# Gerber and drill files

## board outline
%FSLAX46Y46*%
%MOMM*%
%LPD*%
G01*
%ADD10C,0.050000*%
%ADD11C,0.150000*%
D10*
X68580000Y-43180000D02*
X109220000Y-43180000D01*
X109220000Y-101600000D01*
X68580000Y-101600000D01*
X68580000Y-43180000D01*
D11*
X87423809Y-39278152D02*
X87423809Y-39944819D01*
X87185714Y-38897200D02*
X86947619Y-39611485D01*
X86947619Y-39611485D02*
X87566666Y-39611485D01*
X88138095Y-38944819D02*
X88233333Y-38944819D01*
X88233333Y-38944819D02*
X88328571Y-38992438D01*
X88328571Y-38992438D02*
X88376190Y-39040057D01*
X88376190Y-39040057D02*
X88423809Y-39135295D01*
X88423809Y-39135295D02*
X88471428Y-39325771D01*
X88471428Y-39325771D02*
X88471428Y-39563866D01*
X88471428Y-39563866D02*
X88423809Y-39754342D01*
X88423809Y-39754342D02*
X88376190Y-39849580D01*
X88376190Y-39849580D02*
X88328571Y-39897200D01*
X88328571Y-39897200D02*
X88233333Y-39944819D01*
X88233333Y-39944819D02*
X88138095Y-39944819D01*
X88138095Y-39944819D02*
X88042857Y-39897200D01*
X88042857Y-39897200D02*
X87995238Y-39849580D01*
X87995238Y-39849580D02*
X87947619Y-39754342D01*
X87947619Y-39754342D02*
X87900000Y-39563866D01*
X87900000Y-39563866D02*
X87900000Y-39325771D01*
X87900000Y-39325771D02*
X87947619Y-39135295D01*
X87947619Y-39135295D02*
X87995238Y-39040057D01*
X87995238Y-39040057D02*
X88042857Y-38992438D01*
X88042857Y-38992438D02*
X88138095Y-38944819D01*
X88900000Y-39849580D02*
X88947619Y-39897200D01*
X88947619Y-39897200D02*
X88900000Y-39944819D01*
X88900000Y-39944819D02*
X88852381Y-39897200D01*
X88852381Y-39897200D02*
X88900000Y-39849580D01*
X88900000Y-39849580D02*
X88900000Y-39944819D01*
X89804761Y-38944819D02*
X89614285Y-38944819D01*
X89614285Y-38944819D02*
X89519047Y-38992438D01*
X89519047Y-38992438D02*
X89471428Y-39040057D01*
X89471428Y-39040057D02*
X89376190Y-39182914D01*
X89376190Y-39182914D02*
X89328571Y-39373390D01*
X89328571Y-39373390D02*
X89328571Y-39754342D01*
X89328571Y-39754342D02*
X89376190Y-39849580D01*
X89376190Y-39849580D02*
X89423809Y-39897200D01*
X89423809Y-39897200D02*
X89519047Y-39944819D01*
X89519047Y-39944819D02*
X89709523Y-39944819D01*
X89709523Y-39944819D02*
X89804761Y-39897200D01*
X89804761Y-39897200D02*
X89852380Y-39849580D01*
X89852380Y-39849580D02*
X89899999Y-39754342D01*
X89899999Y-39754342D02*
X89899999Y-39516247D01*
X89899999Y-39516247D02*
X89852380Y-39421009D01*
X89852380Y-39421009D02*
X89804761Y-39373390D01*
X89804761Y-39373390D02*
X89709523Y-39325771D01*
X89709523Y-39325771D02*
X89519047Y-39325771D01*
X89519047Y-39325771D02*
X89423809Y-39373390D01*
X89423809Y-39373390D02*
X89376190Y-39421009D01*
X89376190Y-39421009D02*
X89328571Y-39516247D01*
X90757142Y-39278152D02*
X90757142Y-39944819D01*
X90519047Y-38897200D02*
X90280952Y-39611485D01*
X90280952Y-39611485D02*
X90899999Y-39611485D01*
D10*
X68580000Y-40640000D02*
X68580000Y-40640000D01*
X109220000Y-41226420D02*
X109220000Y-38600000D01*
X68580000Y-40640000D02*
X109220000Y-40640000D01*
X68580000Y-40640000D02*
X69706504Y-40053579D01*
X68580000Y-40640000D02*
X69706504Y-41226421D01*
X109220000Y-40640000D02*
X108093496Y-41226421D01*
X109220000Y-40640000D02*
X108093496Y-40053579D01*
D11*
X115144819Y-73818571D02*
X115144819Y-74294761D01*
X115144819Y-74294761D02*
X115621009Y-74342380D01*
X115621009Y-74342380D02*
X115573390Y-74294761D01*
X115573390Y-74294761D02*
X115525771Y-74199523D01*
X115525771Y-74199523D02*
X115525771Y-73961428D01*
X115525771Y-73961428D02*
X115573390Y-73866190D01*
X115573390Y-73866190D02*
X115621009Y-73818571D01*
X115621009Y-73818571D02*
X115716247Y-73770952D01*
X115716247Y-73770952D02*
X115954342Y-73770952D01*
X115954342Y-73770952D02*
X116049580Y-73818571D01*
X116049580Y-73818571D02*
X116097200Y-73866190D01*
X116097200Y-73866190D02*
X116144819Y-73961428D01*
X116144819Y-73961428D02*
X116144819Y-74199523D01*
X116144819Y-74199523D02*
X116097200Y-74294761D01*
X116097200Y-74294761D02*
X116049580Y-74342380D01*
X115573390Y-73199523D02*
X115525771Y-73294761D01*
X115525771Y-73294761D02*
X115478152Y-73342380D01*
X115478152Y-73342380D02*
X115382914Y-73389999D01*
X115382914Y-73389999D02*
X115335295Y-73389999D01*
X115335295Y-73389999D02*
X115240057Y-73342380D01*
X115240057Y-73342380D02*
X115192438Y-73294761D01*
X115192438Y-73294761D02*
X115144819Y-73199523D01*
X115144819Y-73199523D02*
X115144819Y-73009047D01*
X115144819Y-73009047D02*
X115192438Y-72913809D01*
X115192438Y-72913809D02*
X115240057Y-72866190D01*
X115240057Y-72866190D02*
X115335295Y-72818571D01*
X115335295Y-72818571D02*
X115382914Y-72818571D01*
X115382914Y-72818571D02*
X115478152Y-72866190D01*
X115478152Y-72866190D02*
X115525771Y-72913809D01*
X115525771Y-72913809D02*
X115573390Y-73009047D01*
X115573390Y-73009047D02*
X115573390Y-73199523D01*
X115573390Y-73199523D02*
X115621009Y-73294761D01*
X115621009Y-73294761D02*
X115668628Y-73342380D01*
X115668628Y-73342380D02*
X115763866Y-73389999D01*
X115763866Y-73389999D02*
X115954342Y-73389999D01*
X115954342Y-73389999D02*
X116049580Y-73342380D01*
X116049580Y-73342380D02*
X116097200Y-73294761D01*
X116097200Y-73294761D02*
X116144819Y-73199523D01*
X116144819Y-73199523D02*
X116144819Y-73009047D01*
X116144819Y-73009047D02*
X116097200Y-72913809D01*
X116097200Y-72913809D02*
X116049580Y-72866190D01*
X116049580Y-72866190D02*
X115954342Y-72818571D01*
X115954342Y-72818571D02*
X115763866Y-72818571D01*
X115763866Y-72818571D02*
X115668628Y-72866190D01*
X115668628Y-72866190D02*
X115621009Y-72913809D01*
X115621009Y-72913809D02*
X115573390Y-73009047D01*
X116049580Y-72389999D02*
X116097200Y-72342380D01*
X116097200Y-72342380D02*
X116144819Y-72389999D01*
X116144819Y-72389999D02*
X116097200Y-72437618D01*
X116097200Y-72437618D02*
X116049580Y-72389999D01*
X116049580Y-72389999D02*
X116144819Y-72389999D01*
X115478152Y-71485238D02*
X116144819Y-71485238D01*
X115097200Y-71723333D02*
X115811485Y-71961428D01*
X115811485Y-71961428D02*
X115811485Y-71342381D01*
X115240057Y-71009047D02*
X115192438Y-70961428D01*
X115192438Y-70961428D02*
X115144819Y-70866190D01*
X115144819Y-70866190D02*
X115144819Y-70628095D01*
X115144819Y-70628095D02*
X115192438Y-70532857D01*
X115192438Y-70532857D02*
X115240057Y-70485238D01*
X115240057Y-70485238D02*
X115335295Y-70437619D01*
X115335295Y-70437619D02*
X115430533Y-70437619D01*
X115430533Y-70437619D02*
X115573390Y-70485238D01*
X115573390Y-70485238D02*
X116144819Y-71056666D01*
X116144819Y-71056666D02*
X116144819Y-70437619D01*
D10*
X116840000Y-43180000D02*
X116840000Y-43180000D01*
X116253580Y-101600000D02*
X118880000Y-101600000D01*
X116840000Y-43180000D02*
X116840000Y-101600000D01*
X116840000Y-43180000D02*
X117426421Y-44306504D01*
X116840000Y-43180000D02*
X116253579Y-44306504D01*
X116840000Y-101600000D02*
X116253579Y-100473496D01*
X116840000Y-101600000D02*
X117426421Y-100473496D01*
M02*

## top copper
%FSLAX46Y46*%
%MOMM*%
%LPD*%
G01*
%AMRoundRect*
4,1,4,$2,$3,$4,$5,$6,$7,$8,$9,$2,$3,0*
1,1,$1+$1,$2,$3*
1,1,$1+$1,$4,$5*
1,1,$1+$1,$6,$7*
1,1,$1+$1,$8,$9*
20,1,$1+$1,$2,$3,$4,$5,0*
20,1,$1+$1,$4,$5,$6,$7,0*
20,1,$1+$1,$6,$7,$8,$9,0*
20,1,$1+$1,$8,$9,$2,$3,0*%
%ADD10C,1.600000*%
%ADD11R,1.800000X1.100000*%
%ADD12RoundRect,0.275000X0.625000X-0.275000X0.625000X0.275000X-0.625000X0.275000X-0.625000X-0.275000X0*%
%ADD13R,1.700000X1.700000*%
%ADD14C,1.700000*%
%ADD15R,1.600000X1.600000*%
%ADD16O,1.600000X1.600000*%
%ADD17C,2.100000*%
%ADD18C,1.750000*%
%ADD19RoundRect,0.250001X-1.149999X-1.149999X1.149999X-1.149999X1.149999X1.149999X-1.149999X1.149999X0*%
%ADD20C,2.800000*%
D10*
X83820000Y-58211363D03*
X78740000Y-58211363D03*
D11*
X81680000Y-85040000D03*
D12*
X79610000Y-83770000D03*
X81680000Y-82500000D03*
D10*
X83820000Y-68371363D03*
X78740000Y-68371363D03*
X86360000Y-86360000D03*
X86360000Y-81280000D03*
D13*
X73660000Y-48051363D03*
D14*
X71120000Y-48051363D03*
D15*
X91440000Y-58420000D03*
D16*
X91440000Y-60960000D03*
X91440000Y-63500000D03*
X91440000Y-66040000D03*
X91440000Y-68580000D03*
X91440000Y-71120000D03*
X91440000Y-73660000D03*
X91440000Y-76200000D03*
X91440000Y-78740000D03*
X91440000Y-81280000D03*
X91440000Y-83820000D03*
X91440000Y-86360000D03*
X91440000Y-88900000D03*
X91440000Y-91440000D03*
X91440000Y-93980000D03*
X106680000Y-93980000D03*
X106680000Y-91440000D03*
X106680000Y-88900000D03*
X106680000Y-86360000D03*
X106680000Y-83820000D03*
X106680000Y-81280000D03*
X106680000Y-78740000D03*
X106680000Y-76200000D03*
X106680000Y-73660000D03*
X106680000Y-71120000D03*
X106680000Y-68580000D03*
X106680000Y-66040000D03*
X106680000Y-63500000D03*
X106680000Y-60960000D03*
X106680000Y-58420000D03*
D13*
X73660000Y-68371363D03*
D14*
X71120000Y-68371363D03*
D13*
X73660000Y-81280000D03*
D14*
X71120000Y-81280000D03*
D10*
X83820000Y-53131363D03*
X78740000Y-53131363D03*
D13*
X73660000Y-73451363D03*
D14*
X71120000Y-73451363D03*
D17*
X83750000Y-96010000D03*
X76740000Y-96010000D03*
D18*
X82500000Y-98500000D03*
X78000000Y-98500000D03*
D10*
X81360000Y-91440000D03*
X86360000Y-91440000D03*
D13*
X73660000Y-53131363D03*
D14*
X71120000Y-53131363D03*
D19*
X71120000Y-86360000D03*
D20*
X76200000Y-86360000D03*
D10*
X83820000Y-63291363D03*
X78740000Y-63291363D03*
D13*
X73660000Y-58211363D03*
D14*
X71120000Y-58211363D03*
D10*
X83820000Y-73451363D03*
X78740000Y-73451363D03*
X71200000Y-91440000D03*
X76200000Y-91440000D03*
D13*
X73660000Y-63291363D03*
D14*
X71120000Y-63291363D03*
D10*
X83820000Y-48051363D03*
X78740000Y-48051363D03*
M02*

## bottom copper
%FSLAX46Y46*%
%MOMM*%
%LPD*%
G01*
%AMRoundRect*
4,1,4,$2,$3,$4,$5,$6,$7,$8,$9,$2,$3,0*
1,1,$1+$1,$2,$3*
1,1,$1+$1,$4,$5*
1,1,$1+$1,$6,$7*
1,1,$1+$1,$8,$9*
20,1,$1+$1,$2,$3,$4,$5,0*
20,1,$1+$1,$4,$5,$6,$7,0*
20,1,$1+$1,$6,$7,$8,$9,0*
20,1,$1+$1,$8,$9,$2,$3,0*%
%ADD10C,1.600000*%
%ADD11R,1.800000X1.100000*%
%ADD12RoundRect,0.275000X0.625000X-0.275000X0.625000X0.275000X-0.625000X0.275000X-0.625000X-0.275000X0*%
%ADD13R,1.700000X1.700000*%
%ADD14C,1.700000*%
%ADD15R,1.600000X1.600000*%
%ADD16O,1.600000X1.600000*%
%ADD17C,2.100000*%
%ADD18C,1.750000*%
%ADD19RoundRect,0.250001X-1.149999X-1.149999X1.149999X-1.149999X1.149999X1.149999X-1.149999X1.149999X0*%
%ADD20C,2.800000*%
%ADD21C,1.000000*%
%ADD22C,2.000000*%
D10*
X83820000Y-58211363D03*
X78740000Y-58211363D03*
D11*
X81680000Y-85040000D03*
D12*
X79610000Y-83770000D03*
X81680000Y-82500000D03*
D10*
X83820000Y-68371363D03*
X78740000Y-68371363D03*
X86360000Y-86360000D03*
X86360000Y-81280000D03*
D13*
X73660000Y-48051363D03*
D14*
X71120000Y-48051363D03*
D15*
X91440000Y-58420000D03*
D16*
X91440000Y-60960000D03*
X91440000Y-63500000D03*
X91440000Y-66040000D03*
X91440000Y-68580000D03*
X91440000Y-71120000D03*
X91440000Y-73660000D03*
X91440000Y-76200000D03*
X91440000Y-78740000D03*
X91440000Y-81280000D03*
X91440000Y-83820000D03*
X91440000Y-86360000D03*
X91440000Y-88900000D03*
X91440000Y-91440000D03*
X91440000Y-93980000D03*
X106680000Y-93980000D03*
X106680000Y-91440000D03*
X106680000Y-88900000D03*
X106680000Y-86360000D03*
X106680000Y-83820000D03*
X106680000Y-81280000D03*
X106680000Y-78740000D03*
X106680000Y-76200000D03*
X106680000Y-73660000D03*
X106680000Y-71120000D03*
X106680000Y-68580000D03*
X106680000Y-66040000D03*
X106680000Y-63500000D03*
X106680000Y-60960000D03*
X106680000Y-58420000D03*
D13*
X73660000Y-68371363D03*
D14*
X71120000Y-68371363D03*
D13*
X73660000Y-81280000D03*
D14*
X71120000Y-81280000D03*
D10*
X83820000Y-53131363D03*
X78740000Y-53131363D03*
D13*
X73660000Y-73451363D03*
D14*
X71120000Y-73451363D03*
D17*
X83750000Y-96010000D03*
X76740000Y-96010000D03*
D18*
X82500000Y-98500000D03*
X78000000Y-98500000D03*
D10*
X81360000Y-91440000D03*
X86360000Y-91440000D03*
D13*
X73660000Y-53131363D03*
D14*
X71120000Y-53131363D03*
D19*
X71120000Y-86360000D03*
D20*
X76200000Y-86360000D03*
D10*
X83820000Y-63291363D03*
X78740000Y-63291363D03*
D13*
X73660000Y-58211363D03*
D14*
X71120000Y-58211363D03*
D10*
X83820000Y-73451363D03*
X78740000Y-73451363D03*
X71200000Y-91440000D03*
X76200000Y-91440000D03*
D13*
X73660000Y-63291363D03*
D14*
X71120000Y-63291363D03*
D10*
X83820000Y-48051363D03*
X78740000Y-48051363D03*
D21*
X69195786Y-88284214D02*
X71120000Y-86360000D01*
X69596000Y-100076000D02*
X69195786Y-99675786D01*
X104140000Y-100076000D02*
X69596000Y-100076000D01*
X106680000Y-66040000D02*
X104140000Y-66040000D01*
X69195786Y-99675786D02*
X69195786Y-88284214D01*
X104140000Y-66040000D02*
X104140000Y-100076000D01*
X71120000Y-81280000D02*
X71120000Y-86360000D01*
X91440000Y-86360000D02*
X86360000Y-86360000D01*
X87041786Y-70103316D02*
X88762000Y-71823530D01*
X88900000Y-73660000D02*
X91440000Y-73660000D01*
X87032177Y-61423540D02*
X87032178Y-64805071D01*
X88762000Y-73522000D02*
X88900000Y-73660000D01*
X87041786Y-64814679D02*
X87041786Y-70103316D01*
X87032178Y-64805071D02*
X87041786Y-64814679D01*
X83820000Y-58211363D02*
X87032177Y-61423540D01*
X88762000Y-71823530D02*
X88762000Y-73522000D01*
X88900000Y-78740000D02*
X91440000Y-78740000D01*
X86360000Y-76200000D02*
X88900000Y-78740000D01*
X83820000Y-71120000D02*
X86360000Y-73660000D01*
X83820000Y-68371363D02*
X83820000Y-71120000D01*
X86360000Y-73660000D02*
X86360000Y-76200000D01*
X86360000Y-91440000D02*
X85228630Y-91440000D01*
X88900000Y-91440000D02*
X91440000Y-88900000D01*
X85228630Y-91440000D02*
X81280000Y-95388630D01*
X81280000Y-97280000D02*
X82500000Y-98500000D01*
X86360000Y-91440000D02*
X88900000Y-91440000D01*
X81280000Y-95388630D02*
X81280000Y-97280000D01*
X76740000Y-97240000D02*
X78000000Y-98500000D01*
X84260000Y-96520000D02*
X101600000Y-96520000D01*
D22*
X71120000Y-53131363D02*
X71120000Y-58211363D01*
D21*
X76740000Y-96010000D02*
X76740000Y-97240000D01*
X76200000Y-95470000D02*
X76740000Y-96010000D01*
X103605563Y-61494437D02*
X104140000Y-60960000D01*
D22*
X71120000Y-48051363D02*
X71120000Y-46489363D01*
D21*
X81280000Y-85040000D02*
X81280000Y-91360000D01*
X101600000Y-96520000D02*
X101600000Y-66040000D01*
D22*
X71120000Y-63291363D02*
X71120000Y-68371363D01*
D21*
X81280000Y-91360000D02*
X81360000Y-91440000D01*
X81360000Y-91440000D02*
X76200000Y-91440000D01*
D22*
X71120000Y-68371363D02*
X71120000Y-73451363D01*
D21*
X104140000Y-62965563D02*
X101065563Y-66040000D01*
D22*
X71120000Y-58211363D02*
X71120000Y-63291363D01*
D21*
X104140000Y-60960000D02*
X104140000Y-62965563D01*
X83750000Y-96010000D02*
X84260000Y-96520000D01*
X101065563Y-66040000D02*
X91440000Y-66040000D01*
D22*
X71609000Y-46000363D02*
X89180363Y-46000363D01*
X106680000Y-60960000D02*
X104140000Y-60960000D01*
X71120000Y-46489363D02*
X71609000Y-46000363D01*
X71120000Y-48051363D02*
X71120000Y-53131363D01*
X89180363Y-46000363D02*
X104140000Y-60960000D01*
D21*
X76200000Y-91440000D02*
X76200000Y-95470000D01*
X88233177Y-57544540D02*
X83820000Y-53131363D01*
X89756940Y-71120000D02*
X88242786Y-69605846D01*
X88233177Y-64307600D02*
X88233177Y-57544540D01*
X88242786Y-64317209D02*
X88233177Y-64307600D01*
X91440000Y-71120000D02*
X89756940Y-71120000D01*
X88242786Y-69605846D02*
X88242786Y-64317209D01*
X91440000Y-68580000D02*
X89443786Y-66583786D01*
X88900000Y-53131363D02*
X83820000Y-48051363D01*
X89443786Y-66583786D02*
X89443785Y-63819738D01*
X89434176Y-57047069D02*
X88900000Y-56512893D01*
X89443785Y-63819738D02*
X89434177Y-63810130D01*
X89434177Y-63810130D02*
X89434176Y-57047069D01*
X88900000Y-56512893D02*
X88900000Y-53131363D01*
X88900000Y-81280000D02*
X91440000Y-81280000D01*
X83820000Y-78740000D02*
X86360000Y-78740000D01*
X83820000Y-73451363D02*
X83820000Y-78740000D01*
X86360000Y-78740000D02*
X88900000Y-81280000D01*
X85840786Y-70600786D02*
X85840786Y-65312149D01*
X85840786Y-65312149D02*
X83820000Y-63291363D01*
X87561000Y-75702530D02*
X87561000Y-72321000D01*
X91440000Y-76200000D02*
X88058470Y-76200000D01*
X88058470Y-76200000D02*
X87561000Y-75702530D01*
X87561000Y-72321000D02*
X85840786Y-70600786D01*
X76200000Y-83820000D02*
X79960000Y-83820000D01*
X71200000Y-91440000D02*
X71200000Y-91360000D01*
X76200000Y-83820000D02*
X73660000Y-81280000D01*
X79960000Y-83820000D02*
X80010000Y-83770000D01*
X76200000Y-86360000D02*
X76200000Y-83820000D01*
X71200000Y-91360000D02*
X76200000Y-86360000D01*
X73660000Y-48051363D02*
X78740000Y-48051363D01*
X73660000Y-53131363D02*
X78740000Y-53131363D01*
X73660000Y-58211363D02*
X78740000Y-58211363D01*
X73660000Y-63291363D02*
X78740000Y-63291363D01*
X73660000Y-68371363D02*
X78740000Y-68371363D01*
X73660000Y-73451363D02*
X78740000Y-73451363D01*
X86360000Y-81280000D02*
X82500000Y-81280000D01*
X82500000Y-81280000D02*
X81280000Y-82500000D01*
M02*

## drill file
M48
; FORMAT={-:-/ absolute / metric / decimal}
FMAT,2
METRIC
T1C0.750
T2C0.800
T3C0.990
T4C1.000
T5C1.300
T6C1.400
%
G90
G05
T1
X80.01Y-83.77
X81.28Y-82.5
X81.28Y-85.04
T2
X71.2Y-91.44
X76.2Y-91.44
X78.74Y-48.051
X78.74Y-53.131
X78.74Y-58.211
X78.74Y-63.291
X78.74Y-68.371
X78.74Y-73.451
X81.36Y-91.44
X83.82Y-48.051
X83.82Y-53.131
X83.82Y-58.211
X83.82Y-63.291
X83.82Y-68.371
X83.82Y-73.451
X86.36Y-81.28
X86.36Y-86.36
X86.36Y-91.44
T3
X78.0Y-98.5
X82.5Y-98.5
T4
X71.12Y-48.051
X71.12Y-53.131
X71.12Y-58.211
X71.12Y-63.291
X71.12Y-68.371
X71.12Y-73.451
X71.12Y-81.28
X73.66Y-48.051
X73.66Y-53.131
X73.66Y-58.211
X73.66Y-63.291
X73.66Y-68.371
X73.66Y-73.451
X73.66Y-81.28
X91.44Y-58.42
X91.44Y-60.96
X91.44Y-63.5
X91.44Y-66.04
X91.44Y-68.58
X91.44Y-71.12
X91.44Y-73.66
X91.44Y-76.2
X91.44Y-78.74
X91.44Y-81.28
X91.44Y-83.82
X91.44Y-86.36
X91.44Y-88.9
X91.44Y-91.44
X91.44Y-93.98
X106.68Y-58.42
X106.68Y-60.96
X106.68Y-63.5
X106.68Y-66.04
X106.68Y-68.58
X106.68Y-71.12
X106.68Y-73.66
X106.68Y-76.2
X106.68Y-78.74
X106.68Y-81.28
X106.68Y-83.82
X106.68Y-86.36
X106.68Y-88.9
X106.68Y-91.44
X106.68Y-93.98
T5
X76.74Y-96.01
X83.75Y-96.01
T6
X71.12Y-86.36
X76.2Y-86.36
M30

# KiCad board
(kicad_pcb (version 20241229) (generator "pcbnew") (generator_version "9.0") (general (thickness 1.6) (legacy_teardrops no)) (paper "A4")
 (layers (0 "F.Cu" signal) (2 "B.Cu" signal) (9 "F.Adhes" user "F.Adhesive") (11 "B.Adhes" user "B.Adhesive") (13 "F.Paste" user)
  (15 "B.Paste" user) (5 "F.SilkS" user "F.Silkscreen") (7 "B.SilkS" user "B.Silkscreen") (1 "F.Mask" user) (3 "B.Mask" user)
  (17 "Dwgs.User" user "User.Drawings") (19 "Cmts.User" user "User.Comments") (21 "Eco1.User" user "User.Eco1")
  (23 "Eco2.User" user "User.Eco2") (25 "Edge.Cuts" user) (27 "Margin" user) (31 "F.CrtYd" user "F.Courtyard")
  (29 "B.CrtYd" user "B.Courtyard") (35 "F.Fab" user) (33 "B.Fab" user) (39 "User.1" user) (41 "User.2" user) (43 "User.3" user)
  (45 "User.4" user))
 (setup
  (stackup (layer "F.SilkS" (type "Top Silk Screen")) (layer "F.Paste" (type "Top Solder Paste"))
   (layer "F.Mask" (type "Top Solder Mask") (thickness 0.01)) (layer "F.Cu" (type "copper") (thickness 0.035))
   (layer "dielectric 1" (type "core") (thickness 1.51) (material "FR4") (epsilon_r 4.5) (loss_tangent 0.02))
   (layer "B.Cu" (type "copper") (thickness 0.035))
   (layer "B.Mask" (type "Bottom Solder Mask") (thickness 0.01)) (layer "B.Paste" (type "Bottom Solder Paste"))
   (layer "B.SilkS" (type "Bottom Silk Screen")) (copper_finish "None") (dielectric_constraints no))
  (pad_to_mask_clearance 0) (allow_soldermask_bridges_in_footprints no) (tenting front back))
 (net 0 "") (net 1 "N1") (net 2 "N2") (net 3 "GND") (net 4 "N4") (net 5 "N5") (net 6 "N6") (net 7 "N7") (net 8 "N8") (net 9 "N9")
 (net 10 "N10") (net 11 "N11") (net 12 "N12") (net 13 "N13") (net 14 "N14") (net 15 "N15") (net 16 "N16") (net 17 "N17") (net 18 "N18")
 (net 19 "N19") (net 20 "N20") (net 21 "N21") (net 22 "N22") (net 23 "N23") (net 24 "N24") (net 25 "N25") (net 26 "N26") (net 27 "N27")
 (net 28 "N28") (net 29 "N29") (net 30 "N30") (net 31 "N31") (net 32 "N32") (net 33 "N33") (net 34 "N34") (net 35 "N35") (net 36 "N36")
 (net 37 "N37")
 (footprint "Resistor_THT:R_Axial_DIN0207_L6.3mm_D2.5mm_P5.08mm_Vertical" (layer "F.Cu") (at 83.82 58.211363 180)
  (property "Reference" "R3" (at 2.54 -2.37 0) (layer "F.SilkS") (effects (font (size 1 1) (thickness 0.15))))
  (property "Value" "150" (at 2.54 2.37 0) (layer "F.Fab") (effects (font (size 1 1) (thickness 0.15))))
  (pad "1" thru_hole circle (at 0 0 180) (size 1.6 1.6) (drill 0.8) (layers "*.Cu" "*.Mask") (remove_unused_layers no) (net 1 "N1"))
  (pad "2" thru_hole circle (at 5.08 0 180) (size 1.6 1.6) (drill 0.8) (layers "*.Cu" "*.Mask") (remove_unused_layers no) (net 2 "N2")))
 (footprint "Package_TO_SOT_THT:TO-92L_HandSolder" (layer "F.Cu") (at 81.28 85.04 90)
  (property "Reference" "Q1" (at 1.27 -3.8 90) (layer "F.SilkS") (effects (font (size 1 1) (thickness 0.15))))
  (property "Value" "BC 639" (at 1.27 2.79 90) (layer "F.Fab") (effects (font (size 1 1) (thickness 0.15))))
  (pad "1" thru_hole rect (at 0 0 90) (size 1.1 1.8) (drill 0.75 (offset 0 0.4)) (layers "*.Cu" "*.Mask") (remove_unused_layers no)
   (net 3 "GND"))
  (pad "2" thru_hole roundrect (at 1.27 -1.27 90) (size 1.1 1.8) (drill 0.75 (offset 0 -0.4)) (layers "*.Cu" "*.Mask")
   (remove_unused_layers no) (roundrect_rratio 0.25) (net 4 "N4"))
  (pad "3" thru_hole roundrect (at 2.54 0 90) (size 1.1 1.8) (drill 0.75 (offset 0 0.4)) (layers "*.Cu" "*.Mask") (remove_unused_layers no)
   (roundrect_rratio 0.25) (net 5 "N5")))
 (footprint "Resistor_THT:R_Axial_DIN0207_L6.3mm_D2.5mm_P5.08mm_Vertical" (layer "F.Cu") (at 83.82 68.371363 180)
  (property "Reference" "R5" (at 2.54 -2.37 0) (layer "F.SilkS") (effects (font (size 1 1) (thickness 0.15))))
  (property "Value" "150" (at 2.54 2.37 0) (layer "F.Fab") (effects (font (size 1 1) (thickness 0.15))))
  (pad "1" thru_hole circle (at 0 0 180) (size 1.6 1.6) (drill 0.8) (layers "*.Cu" "*.Mask") (remove_unused_layers no) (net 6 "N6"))
  (pad "2" thru_hole circle (at 5.08 0 180) (size 1.6 1.6) (drill 0.8) (layers "*.Cu" "*.Mask") (remove_unused_layers no) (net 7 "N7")))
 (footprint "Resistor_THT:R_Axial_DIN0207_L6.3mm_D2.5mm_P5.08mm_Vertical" (layer "F.Cu") (at 86.36 86.36 90)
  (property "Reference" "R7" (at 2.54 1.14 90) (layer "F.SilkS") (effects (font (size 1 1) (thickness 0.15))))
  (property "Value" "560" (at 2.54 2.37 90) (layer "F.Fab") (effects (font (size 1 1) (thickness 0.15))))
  (pad "1" thru_hole circle (at 0 0 90) (size 1.6 1.6) (drill 0.8) (layers "*.Cu" "*.Mask") (remove_unused_layers no) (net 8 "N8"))
  (pad "2" thru_hole circle (at 5.08 0 90) (size 1.6 1.6) (drill 0.8) (layers "*.Cu" "*.Mask") (remove_unused_layers no) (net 5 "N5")))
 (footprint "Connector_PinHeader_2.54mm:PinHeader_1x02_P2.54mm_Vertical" (layer "F.Cu") (at 73.66 48.051363 -90)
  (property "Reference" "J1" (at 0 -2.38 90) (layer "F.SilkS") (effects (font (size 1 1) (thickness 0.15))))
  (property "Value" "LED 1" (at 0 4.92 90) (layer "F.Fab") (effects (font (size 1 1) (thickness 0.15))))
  (pad "1" thru_hole rect (at 0 0 270) (size 1.7 1.7) (drill 1) (layers "*.Cu" "*.Mask") (remove_unused_layers no) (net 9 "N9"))
  (pad "2" thru_hole circle (at 0 2.54 270) (size 1.7 1.7) (drill 1) (layers "*.Cu" "*.Mask") (remove_unused_layers no) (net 3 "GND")))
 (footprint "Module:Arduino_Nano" (layer "F.Cu") (at 91.44 58.42)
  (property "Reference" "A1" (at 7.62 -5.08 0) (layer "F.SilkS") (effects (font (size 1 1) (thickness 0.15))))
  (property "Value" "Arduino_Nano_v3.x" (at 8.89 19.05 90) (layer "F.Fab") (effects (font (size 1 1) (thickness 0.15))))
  (pad "1" thru_hole rect (at 0 0) (size 1.6 1.6) (drill 1) (layers "*.Cu" "*.Mask") (remove_unused_layers no) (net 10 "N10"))
  (pad "2" thru_hole oval (at 0 2.54) (size 1.6 1.6) (drill 1) (layers "*.Cu" "*.Mask") (remove_unused_layers no) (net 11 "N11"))
  (pad "3" thru_hole oval (at 0 5.08) (size 1.6 1.6) (drill 1) (layers "*.Cu" "*.Mask") (remove_unused_layers no) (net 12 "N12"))
  (pad "4" thru_hole oval (at 0 7.62) (size 1.6 1.6) (drill 1) (layers "*.Cu" "*.Mask") (remove_unused_layers no) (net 3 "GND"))
  (pad "5" thru_hole oval (at 0 10.16) (size 1.6 1.6) (drill 1) (layers "*.Cu" "*.Mask") (remove_unused_layers no) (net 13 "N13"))
  (pad "6" thru_hole oval (at 0 12.7) (size 1.6 1.6) (drill 1) (layers "*.Cu" "*.Mask") (remove_unused_layers no) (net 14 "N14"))
  (pad "7" thru_hole oval (at 0 15.24) (size 1.6 1.6) (drill 1) (layers "*.Cu" "*.Mask") (remove_unused_layers no) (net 1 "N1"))
  (pad "8" thru_hole oval (at 0 17.78) (size 1.6 1.6) (drill 1) (layers "*.Cu" "*.Mask") (remove_unused_layers no) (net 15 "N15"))
  (pad "9" thru_hole oval (at 0 20.32) (size 1.6 1.6) (drill 1) (layers "*.Cu" "*.Mask") (remove_unused_layers no) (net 6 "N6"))
  (pad "10" thru_hole oval (at 0 22.86) (size 1.6 1.6) (drill 1) (layers "*.Cu" "*.Mask") (remove_unused_layers no) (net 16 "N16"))
  (pad "11" thru_hole oval (at 0 25.4) (size 1.6 1.6) (drill 1) (layers "*.Cu" "*.Mask") (remove_unused_layers no) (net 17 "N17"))
  (pad "12" thru_hole oval (at 0 27.94) (size 1.6 1.6) (drill 1) (layers "*.Cu" "*.Mask") (remove_unused_layers no) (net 8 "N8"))
  (pad "13" thru_hole oval (at 0 30.48) (size 1.6 1.6) (drill 1) (layers "*.Cu" "*.Mask") (remove_unused_layers no) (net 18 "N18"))
  (pad "14" thru_hole oval (at 0 33.02) (size 1.6 1.6) (drill 1) (layers "*.Cu" "*.Mask") (remove_unused_layers no) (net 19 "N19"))
  (pad "15" thru_hole oval (at 0 35.56) (size 1.6 1.6) (drill 1) (layers "*.Cu" "*.Mask") (remove_unused_layers no) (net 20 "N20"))
  (pad "16" thru_hole oval (at 15.24 35.56) (size 1.6 1.6) (drill 1) (layers "*.Cu" "*.Mask") (remove_unused_layers no) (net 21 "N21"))
  (pad "17" thru_hole oval (at 15.24 33.02) (size 1.6 1.6) (drill 1) (layers "*.Cu" "*.Mask") (remove_unused_layers no) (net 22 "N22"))
  (pad "18" thru_hole oval (at 15.24 30.48) (size 1.6 1.6) (drill 1) (layers "*.Cu" "*.Mask") (remove_unused_layers no) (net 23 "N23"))
  (pad "19" thru_hole oval (at 15.24 27.94) (size 1.6 1.6) (drill 1) (layers "*.Cu" "*.Mask") (remove_unused_layers no) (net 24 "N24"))
  (pad "20" thru_hole oval (at 15.24 25.4) (size 1.6 1.6) (drill 1) (layers "*.Cu" "*.Mask") (remove_unused_layers no) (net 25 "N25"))
  (pad "21" thru_hole oval (at 15.24 22.86) (size 1.6 1.6) (drill 1) (layers "*.Cu" "*.Mask") (remove_unused_layers no) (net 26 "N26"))
  (pad "22" thru_hole oval (at 15.24 20.32) (size 1.6 1.6) (drill 1) (layers "*.Cu" "*.Mask") (remove_unused_layers no) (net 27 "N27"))
  (pad "23" thru_hole oval (at 15.24 17.78) (size 1.6 1.6) (drill 1) (layers "*.Cu" "*.Mask") (remove_unused_layers no) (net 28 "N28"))
  (pad "24" thru_hole oval (at 15.24 15.24) (size 1.6 1.6) (drill 1) (layers "*.Cu" "*.Mask") (remove_unused_layers no) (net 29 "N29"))
  (pad "25" thru_hole oval (at 15.24 12.7) (size 1.6 1.6) (drill 1) (layers "*.Cu" "*.Mask") (remove_unused_layers no) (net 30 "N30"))
  (pad "26" thru_hole oval (at 15.24 10.16) (size 1.6 1.6) (drill 1) (layers "*.Cu" "*.Mask") (remove_unused_layers no) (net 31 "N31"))
  (pad "27" thru_hole oval (at 15.24 7.62) (size 1.6 1.6) (drill 1) (layers "*.Cu" "*.Mask") (remove_unused_layers no) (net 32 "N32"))
  (pad "28" thru_hole oval (at 15.24 5.08) (size 1.6 1.6) (drill 1) (layers "*.Cu" "*.Mask") (remove_unused_layers no) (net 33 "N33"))
  (pad "29" thru_hole oval (at 15.24 2.54) (size 1.6 1.6) (drill 1) (layers "*.Cu" "*.Mask") (remove_unused_layers no) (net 3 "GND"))
  (pad "30" thru_hole oval (at 15.24 0) (size 1.6 1.6) (drill 1) (layers "*.Cu" "*.Mask") (remove_unused_layers no) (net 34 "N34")))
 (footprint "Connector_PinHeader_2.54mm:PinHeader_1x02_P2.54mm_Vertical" (layer "F.Cu") (at 73.66 68.371363 -90)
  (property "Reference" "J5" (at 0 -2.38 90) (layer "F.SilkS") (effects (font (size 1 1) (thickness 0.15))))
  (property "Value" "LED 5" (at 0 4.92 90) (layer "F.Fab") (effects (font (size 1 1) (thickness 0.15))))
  (pad "1" thru_hole rect (at 0 0 270) (size 1.7 1.7) (drill 1) (layers "*.Cu" "*.Mask") (remove_unused_layers no) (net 7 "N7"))
  (pad "2" thru_hole circle (at 0 2.54 270) (size 1.7 1.7) (drill 1) (layers "*.Cu" "*.Mask") (remove_unused_layers no) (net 3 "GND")))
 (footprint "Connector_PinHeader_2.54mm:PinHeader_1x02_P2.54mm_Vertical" (layer "F.Cu") (at 73.66 81.28 -90)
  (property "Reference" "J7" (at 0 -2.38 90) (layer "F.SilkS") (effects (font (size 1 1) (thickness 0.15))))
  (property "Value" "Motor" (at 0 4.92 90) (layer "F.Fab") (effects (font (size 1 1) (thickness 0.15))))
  (pad "1" thru_hole rect (at 0 0 270) (size 1.7 1.7) (drill 1) (layers "*.Cu" "*.Mask") (remove_unused_layers no) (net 4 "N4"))
  (pad "2" thru_hole circle (at 0 2.54 270) (size 1.7 1.7) (drill 1) (layers "*.Cu" "*.Mask") (remove_unused_layers no) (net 32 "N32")))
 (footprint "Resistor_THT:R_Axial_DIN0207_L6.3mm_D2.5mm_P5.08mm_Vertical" (layer "F.Cu") (at 83.82 53.131363 180)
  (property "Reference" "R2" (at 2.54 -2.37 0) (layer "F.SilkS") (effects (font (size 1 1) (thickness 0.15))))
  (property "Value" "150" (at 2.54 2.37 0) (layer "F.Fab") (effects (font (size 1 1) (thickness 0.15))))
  (pad "1" thru_hole circle (at 0 0 180) (size 1.6 1.6) (drill 0.8) (layers "*.Cu" "*.Mask") (remove_unused_layers no) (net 14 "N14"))
  (pad "2" thru_hole circle (at 5.08 0 180) (size 1.6 1.6) (drill 0.8) (layers "*.Cu" "*.Mask") (remove_unused_layers no) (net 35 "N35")))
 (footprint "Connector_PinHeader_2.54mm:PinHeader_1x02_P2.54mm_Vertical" (layer "F.Cu") (at 73.66 73.451363 -90)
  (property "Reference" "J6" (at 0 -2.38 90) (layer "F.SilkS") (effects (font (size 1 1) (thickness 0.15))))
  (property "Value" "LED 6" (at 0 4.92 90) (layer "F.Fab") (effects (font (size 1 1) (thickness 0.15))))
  (pad "1" thru_hole rect (at 0 0 270) (size 1.7 1.7) (drill 1) (layers "*.Cu" "*.Mask") (remove_unused_layers no) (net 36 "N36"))
  (pad "2" thru_hole circle (at 0 2.54 270) (size 1.7 1.7) (drill 1) (layers "*.Cu" "*.Mask") (remove_unused_layers no) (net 3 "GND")))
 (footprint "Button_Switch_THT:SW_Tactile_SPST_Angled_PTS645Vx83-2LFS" (layer "F.Cu") (at 82.5 98.5 180)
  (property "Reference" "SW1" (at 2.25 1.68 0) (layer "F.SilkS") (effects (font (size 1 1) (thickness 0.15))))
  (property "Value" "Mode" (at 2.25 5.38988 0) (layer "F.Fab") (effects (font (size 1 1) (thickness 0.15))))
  (pad "" thru_hole circle (at -1.25 2.49 180) (size 2.1 2.1) (drill 1.3) (layers "*.Cu" "*.Mask") (remove_unused_layers no))
  (pad "" thru_hole circle (at 5.76 2.49 180) (size 2.1 2.1) (drill 1.3) (layers "*.Cu" "*.Mask") (remove_unused_layers no))
  (pad "1" thru_hole circle (at 0 0 180) (size 1.75 1.75) (drill 0.99) (layers "*.Cu" "*.Mask") (remove_unused_layers no) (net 18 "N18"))
  (pad "2" thru_hole circle (at 4.5 0 180) (size 1.75 1.75) (drill 0.99) (layers "*.Cu" "*.Mask") (remove_unused_layers no) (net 3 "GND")))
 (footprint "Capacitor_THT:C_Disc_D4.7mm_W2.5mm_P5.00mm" (layer "F.Cu") (at 81.36 91.44)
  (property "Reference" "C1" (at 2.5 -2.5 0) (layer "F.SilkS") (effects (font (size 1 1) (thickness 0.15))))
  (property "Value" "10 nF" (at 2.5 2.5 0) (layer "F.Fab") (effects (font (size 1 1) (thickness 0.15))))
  (pad "1" thru_hole circle (at 0 0) (size 1.6 1.6) (drill 0.8) (layers "*.Cu" "*.Mask") (remove_unused_layers no) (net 3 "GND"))
  (pad "2" thru_hole circle (at 5 0) (size 1.6 1.6) (drill 0.8) (layers "*.Cu" "*.Mask") (remove_unused_layers no) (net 18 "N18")))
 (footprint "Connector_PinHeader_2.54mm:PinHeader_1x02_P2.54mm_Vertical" (layer "F.Cu") (at 73.66 53.131363 -90)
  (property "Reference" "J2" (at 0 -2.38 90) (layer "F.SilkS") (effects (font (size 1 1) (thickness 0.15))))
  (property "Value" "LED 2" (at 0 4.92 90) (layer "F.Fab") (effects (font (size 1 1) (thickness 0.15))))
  (pad "1" thru_hole rect (at 0 0 270) (size 1.7 1.7) (drill 1) (layers "*.Cu" "*.Mask") (remove_unused_layers no) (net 35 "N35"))
  (pad "2" thru_hole circle (at 0 2.54 270) (size 1.7 1.7) (drill 1) (layers "*.Cu" "*.Mask") (remove_unused_layers no) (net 3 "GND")))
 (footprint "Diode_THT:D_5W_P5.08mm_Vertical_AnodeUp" (layer "F.Cu") (at 71.12 86.36)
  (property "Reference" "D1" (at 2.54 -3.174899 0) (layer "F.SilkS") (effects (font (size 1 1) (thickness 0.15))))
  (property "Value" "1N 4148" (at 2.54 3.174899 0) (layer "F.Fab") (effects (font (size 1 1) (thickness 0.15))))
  (pad "1" thru_hole roundrect (at 0 0) (size 2.8 2.8) (drill 1.4) (layers "*.Cu" "*.Mask") (remove_unused_layers no)
   (roundrect_rratio 0.089286) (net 32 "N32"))
  (pad "2" thru_hole circle (at 5.08 0) (size 2.8 2.8) (drill 1.4) (layers "*.Cu" "*.Mask") (remove_unused_layers no) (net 4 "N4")))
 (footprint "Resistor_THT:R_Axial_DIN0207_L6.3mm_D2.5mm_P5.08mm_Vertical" (layer "F.Cu") (at 83.82 63.291363 180)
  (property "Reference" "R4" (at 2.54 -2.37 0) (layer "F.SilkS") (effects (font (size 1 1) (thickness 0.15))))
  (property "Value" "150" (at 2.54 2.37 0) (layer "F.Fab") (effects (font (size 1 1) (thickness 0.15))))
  (pad "1" thru_hole circle (at 0 0 180) (size 1.6 1.6) (drill 0.8) (layers "*.Cu" "*.Mask") (remove_unused_layers no) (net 15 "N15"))
  (pad "2" thru_hole circle (at 5.08 0 180) (size 1.6 1.6) (drill 0.8) (layers "*.Cu" "*.Mask") (remove_unused_layers no) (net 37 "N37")))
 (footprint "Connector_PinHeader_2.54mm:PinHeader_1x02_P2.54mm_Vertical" (layer "F.Cu") (at 73.66 58.211363 -90)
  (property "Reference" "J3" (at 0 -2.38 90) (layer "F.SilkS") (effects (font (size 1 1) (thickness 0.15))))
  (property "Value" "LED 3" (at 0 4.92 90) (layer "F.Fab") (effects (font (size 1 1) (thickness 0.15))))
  (pad "1" thru_hole rect (at 0 0 270) (size 1.7 1.7) (drill 1) (layers "*.Cu" "*.Mask") (remove_unused_layers no) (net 2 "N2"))
  (pad "2" thru_hole circle (at 0 2.54 270) (size 1.7 1.7) (drill 1) (layers "*.Cu" "*.Mask") (remove_unused_layers no) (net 3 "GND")))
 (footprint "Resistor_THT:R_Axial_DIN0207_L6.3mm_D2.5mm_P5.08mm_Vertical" (layer "F.Cu") (at 83.82 73.451363 180)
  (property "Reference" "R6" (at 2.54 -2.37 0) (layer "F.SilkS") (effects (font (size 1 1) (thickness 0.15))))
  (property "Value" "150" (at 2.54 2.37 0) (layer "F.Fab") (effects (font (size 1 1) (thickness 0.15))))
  (pad "1" thru_hole circle (at 0 0 180) (size 1.6 1.6) (drill 0.8) (layers "*.Cu" "*.Mask") (remove_unused_layers no) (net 16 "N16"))
  (pad "2" thru_hole circle (at 5.08 0 180) (size 1.6 1.6) (drill 0.8) (layers "*.Cu" "*.Mask") (remove_unused_layers no) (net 36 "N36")))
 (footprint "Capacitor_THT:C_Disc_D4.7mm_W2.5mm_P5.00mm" (layer "F.Cu") (at 71.2 91.44)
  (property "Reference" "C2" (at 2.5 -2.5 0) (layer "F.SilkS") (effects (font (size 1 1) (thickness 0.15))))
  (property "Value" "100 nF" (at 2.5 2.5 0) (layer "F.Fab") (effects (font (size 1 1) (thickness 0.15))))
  (pad "1" thru_hole circle (at 0 0) (size 1.6 1.6) (drill 0.8) (layers "*.Cu" "*.Mask") (remove_unused_layers no) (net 4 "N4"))
  (pad "2" thru_hole circle (at 5 0) (size 1.6 1.6) (drill 0.8) (layers "*.Cu" "*.Mask") (remove_unused_layers no) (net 3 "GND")))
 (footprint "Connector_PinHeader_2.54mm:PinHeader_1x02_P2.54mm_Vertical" (layer "F.Cu") (at 73.66 63.291363 -90)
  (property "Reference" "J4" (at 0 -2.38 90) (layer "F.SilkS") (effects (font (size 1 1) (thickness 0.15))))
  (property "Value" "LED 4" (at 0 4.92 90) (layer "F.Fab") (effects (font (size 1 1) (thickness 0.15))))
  (pad "1" thru_hole rect (at 0 0 270) (size 1.7 1.7) (drill 1) (layers "*.Cu" "*.Mask") (remove_unused_layers no) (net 37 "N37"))
  (pad "2" thru_hole circle (at 0 2.54 270) (size 1.7 1.7) (drill 1) (layers "*.Cu" "*.Mask") (remove_unused_layers no) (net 3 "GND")))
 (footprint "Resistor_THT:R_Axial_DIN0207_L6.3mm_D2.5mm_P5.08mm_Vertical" (layer "F.Cu") (at 83.82 48.051363 180)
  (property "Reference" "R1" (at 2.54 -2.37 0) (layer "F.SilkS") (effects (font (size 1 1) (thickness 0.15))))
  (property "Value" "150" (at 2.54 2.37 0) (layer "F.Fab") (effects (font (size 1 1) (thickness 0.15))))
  (pad "1" thru_hole circle (at 0 0 180) (size 1.6 1.6) (drill 0.8) (layers "*.Cu" "*.Mask") (remove_unused_layers no) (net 13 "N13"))
  (pad "2" thru_hole circle (at 5.08 0 180) (size 1.6 1.6) (drill 0.8) (layers "*.Cu" "*.Mask") (remove_unused_layers no) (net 9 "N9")))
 (gr_rect (start 68.58 43.18) (end 109.22 101.6) (stroke (width 0.05) (type default)) (fill no) (layer "Edge.Cuts"))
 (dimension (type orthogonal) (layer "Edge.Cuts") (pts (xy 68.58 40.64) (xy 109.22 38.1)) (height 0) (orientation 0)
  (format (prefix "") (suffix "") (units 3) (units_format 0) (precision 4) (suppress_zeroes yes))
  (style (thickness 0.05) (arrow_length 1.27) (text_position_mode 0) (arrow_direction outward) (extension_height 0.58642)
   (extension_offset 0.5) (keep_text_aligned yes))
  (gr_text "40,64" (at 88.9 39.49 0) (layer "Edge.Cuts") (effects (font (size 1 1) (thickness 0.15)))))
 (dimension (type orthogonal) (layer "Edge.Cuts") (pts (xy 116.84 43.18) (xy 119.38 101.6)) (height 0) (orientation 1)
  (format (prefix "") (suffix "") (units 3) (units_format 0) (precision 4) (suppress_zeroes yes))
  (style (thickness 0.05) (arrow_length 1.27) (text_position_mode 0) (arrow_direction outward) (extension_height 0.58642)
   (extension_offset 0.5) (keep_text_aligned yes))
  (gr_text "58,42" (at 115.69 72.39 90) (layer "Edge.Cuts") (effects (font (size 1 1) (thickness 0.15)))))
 (segment (start 69.195786 88.284214) (end 71.12 86.36) (width 1) (layer "B.Cu") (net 32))
 (segment (start 69.596 100.076) (end 69.195786 99.675786) (width 1) (layer "B.Cu") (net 32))
 (segment (start 104.14 100.076) (end 69.596 100.076) (width 1) (layer "B.Cu") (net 32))
 (segment (start 106.68 66.04) (end 104.14 66.04) (width 1) (layer "B.Cu") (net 32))
 (segment (start 69.195786 99.675786) (end 69.195786 88.284214) (width 1) (layer "B.Cu") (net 32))
 (segment (start 104.14 66.04) (end 104.14 100.076) (width 1) (layer "B.Cu") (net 32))
 (segment (start 71.12 81.28) (end 71.12 86.36) (width 1) (layer "B.Cu") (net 32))
 (segment (start 91.44 86.36) (end 86.36 86.36) (width 1) (layer "B.Cu") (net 8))
 (segment (start 87.041786 70.103316) (end 88.762 71.82353) (width 1) (layer "B.Cu") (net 1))
 (segment (start 88.9 73.66) (end 91.44 73.66) (width 1) (layer "B.Cu") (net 1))
 (segment (start 87.032177 61.42354) (end 87.032178 64.805071) (width 1) (layer "B.Cu") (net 1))
 (segment (start 88.762 73.522) (end 88.9 73.66) (width 1) (layer "B.Cu") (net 1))
 (segment (start 87.041786 64.814679) (end 87.041786 70.103316) (width 1) (layer "B.Cu") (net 1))
 (segment (start 87.032178 64.805071) (end 87.041786 64.814679) (width 1) (layer "B.Cu") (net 1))
 (segment (start 83.82 58.211363) (end 87.032177 61.42354) (width 1) (layer "B.Cu") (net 1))
 (segment (start 88.762 71.82353) (end 88.762 73.522) (width 1) (layer "B.Cu") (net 1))
 (segment (start 88.9 78.74) (end 91.44 78.74) (width 1) (layer "B.Cu") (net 6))
 (segment (start 86.36 76.2) (end 88.9 78.74) (width 1) (layer "B.Cu") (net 6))
 (segment (start 83.82 71.12) (end 86.36 73.66) (width 1) (layer "B.Cu") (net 6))
 (segment (start 83.82 68.371363) (end 83.82 71.12) (width 1) (layer "B.Cu") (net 6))
 (segment (start 86.36 73.66) (end 86.36 76.2) (width 1) (layer "B.Cu") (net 6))
 (segment (start 86.36 91.44) (end 85.22863 91.44) (width 1) (layer "B.Cu") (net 18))
 (segment (start 88.9 91.44) (end 91.44 88.9) (width 1) (layer "B.Cu") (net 18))
 (segment (start 85.22863 91.44) (end 81.28 95.38863) (width 1) (layer "B.Cu") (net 18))
 (segment (start 81.28 97.28) (end 82.5 98.5) (width 1) (layer "B.Cu") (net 18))
 (segment (start 86.36 91.44) (end 88.9 91.44) (width 1) (layer "B.Cu") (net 18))
 (segment (start 81.28 95.38863) (end 81.28 97.28) (width 1) (layer "B.Cu") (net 18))
 (segment (start 76.74 97.24) (end 78 98.5) (width 1) (layer "B.Cu") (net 3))
 (segment (start 84.26 96.52) (end 101.6 96.52) (width 1) (layer "B.Cu") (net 3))
 (segment (start 71.12 53.131363) (end 71.12 58.211363) (width 2) (layer "B.Cu") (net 3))
 (segment (start 76.74 96.01) (end 76.74 97.24) (width 1) (layer "B.Cu") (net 3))
 (segment (start 76.2 95.47) (end 76.74 96.01) (width 1) (layer "B.Cu") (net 3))
 (segment (start 103.605563 61.494437) (end 104.14 60.96) (width 1) (layer "B.Cu") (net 3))
 (segment (start 71.12 48.051363) (end 71.12 46.489363) (width 2) (layer "B.Cu") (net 3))
 (segment (start 81.28 85.04) (end 81.28 91.36) (width 1) (layer "B.Cu") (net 3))
 (segment (start 101.6 96.52) (end 101.6 66.04) (width 1) (layer "B.Cu") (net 3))
 (segment (start 71.12 63.291363) (end 71.12 68.371363) (width 2) (layer "B.Cu") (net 3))
 (segment (start 81.28 91.36) (end 81.36 91.44) (width 1) (layer "B.Cu") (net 3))
 (segment (start 81.36 91.44) (end 76.2 91.44) (width 1) (layer "B.Cu") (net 3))
 (segment (start 71.12 68.371363) (end 71.12 73.451363) (width 2) (layer "B.Cu") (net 3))
 (segment (start 104.14 62.965563) (end 101.065563 66.04) (width 1) (layer "B.Cu") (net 3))
 (segment (start 71.12 58.211363) (end 71.12 63.291363) (width 2) (layer "B.Cu") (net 3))
 (segment (start 104.14 60.96) (end 104.14 62.965563) (width 1) (layer "B.Cu") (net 3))
 (segment (start 83.75 96.01) (end 84.26 96.52) (width 1) (layer "B.Cu") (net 3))
 (segment (start 101.065563 66.04) (end 91.44 66.04) (width 1) (layer "B.Cu") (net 3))
 (segment (start 71.609 46.000363) (end 89.180363 46.000363) (width 2) (layer "B.Cu") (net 3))
 (segment (start 106.68 60.96) (end 104.14 60.96) (width 2) (layer "B.Cu") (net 3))
 (segment (start 71.12 46.489363) (end 71.609 46.000363) (width 2) (layer "B.Cu") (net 3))
 (segment (start 71.12 48.051363) (end 71.12 53.131363) (width 2) (layer "B.Cu") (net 3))
 (segment (start 89.180363 46.000363) (end 104.14 60.96) (width 2) (layer "B.Cu") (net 3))
 (segment (start 76.2 91.44) (end 76.2 95.47) (width 1) (layer "B.Cu") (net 3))
 (segment (start 88.233177 57.54454) (end 83.82 53.131363) (width 1) (layer "B.Cu") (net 14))
 (segment (start 89.75694 71.12) (end 88.242786 69.605846) (width 1) (layer "B.Cu") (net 14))
 (segment (start 88.233177 64.3076) (end 88.233177 57.54454) (width 1) (layer "B.Cu") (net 14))
 (segment (start 88.242786 64.317209) (end 88.233177 64.3076) (width 1) (layer "B.Cu") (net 14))
 (segment (start 91.44 71.12) (end 89.75694 71.12) (width 1) (layer "B.Cu") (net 14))
 (segment (start 88.242786 69.605846) (end 88.242786 64.317209) (width 1) (layer "B.Cu") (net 14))
 (segment (start 91.44 68.58) (end 89.443786 66.583786) (width 1) (layer "B.Cu") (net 13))
 (segment (start 88.9 53.131363) (end 83.82 48.051363) (width 1) (layer "B.Cu") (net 13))
 (segment (start 89.443786 66.583786) (end 89.443785 63.819738) (width 1) (layer "B.Cu") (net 13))
 (segment (start 89.434176 57.047069) (end 88.9 56.512893) (width 1) (layer "B.Cu") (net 13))
 (segment (start 89.443785 63.819738) (end 89.434177 63.81013) (width 1) (layer "B.Cu") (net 13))
 (segment (start 89.434177 63.81013) (end 89.434176 57.047069) (width 1) (layer "B.Cu") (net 13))
 (segment (start 88.9 56.512893) (end 88.9 53.131363) (width 1) (layer "B.Cu") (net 13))
 (segment (start 88.9 81.28) (end 91.44 81.28) (width 1) (layer "B.Cu") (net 16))
 (segment (start 83.82 78.74) (end 86.36 78.74) (width 1) (layer "B.Cu") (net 16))
 (segment (start 83.82 73.451363) (end 83.82 78.74) (width 1) (layer "B.Cu") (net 16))
 (segment (start 86.36 78.74) (end 88.9 81.28) (width 1) (layer "B.Cu") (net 16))
 (segment (start 85.840786 70.600786) (end 85.840786 65.312149) (width 1) (layer "B.Cu") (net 15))
 (segment (start 85.840786 65.312149) (end 83.82 63.291363) (width 1) (layer "B.Cu") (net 15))
 (segment (start 87.561 75.70253) (end 87.561 72.321) (width 1) (layer "B.Cu") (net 15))
 (segment (start 91.44 76.2) (end 88.05847 76.2) (width 1) (layer "B.Cu") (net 15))
 (segment (start 88.05847 76.2) (end 87.561 75.70253) (width 1) (layer "B.Cu") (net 15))
 (segment (start 87.561 72.321) (end 85.840786 70.600786) (width 1) (layer "B.Cu") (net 15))
 (segment (start 76.2 83.82) (end 79.96 83.82) (width 1) (layer "B.Cu") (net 4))
 (segment (start 71.2 91.44) (end 71.2 91.36) (width 1) (layer "B.Cu") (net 4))
 (segment (start 76.2 83.82) (end 73.66 81.28) (width 1) (layer "B.Cu") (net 4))
 (segment (start 79.96 83.82) (end 80.01 83.77) (width 1) (layer "B.Cu") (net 4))
 (segment (start 76.2 86.36) (end 76.2 83.82) (width 1) (layer "B.Cu") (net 4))
 (segment (start 71.2 91.36) (end 76.2 86.36) (width 1) (layer "B.Cu") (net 4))
 (segment (start 73.66 48.051363) (end 78.74 48.051363) (width 1) (layer "B.Cu") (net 9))
 (segment (start 73.66 53.131363) (end 78.74 53.131363) (width 1) (layer "B.Cu") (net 35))
 (segment (start 73.66 58.211363) (end 78.74 58.211363) (width 1) (layer "B.Cu") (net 2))
 (segment (start 73.66 63.291363) (end 78.74 63.291363) (width 1) (layer "B.Cu") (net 37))
 (segment (start 73.66 68.371363) (end 78.74 68.371363) (width 1) (layer "B.Cu") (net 7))
 (segment (start 73.66 73.451363) (end 78.74 73.451363) (width 1) (layer "B.Cu") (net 36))
 (segment (start 86.36 81.28) (end 82.5 81.28) (width 1) (layer "B.Cu") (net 5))
 (segment (start 82.5 81.28) (end 81.28 82.5) (width 1) (layer "B.Cu") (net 5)))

